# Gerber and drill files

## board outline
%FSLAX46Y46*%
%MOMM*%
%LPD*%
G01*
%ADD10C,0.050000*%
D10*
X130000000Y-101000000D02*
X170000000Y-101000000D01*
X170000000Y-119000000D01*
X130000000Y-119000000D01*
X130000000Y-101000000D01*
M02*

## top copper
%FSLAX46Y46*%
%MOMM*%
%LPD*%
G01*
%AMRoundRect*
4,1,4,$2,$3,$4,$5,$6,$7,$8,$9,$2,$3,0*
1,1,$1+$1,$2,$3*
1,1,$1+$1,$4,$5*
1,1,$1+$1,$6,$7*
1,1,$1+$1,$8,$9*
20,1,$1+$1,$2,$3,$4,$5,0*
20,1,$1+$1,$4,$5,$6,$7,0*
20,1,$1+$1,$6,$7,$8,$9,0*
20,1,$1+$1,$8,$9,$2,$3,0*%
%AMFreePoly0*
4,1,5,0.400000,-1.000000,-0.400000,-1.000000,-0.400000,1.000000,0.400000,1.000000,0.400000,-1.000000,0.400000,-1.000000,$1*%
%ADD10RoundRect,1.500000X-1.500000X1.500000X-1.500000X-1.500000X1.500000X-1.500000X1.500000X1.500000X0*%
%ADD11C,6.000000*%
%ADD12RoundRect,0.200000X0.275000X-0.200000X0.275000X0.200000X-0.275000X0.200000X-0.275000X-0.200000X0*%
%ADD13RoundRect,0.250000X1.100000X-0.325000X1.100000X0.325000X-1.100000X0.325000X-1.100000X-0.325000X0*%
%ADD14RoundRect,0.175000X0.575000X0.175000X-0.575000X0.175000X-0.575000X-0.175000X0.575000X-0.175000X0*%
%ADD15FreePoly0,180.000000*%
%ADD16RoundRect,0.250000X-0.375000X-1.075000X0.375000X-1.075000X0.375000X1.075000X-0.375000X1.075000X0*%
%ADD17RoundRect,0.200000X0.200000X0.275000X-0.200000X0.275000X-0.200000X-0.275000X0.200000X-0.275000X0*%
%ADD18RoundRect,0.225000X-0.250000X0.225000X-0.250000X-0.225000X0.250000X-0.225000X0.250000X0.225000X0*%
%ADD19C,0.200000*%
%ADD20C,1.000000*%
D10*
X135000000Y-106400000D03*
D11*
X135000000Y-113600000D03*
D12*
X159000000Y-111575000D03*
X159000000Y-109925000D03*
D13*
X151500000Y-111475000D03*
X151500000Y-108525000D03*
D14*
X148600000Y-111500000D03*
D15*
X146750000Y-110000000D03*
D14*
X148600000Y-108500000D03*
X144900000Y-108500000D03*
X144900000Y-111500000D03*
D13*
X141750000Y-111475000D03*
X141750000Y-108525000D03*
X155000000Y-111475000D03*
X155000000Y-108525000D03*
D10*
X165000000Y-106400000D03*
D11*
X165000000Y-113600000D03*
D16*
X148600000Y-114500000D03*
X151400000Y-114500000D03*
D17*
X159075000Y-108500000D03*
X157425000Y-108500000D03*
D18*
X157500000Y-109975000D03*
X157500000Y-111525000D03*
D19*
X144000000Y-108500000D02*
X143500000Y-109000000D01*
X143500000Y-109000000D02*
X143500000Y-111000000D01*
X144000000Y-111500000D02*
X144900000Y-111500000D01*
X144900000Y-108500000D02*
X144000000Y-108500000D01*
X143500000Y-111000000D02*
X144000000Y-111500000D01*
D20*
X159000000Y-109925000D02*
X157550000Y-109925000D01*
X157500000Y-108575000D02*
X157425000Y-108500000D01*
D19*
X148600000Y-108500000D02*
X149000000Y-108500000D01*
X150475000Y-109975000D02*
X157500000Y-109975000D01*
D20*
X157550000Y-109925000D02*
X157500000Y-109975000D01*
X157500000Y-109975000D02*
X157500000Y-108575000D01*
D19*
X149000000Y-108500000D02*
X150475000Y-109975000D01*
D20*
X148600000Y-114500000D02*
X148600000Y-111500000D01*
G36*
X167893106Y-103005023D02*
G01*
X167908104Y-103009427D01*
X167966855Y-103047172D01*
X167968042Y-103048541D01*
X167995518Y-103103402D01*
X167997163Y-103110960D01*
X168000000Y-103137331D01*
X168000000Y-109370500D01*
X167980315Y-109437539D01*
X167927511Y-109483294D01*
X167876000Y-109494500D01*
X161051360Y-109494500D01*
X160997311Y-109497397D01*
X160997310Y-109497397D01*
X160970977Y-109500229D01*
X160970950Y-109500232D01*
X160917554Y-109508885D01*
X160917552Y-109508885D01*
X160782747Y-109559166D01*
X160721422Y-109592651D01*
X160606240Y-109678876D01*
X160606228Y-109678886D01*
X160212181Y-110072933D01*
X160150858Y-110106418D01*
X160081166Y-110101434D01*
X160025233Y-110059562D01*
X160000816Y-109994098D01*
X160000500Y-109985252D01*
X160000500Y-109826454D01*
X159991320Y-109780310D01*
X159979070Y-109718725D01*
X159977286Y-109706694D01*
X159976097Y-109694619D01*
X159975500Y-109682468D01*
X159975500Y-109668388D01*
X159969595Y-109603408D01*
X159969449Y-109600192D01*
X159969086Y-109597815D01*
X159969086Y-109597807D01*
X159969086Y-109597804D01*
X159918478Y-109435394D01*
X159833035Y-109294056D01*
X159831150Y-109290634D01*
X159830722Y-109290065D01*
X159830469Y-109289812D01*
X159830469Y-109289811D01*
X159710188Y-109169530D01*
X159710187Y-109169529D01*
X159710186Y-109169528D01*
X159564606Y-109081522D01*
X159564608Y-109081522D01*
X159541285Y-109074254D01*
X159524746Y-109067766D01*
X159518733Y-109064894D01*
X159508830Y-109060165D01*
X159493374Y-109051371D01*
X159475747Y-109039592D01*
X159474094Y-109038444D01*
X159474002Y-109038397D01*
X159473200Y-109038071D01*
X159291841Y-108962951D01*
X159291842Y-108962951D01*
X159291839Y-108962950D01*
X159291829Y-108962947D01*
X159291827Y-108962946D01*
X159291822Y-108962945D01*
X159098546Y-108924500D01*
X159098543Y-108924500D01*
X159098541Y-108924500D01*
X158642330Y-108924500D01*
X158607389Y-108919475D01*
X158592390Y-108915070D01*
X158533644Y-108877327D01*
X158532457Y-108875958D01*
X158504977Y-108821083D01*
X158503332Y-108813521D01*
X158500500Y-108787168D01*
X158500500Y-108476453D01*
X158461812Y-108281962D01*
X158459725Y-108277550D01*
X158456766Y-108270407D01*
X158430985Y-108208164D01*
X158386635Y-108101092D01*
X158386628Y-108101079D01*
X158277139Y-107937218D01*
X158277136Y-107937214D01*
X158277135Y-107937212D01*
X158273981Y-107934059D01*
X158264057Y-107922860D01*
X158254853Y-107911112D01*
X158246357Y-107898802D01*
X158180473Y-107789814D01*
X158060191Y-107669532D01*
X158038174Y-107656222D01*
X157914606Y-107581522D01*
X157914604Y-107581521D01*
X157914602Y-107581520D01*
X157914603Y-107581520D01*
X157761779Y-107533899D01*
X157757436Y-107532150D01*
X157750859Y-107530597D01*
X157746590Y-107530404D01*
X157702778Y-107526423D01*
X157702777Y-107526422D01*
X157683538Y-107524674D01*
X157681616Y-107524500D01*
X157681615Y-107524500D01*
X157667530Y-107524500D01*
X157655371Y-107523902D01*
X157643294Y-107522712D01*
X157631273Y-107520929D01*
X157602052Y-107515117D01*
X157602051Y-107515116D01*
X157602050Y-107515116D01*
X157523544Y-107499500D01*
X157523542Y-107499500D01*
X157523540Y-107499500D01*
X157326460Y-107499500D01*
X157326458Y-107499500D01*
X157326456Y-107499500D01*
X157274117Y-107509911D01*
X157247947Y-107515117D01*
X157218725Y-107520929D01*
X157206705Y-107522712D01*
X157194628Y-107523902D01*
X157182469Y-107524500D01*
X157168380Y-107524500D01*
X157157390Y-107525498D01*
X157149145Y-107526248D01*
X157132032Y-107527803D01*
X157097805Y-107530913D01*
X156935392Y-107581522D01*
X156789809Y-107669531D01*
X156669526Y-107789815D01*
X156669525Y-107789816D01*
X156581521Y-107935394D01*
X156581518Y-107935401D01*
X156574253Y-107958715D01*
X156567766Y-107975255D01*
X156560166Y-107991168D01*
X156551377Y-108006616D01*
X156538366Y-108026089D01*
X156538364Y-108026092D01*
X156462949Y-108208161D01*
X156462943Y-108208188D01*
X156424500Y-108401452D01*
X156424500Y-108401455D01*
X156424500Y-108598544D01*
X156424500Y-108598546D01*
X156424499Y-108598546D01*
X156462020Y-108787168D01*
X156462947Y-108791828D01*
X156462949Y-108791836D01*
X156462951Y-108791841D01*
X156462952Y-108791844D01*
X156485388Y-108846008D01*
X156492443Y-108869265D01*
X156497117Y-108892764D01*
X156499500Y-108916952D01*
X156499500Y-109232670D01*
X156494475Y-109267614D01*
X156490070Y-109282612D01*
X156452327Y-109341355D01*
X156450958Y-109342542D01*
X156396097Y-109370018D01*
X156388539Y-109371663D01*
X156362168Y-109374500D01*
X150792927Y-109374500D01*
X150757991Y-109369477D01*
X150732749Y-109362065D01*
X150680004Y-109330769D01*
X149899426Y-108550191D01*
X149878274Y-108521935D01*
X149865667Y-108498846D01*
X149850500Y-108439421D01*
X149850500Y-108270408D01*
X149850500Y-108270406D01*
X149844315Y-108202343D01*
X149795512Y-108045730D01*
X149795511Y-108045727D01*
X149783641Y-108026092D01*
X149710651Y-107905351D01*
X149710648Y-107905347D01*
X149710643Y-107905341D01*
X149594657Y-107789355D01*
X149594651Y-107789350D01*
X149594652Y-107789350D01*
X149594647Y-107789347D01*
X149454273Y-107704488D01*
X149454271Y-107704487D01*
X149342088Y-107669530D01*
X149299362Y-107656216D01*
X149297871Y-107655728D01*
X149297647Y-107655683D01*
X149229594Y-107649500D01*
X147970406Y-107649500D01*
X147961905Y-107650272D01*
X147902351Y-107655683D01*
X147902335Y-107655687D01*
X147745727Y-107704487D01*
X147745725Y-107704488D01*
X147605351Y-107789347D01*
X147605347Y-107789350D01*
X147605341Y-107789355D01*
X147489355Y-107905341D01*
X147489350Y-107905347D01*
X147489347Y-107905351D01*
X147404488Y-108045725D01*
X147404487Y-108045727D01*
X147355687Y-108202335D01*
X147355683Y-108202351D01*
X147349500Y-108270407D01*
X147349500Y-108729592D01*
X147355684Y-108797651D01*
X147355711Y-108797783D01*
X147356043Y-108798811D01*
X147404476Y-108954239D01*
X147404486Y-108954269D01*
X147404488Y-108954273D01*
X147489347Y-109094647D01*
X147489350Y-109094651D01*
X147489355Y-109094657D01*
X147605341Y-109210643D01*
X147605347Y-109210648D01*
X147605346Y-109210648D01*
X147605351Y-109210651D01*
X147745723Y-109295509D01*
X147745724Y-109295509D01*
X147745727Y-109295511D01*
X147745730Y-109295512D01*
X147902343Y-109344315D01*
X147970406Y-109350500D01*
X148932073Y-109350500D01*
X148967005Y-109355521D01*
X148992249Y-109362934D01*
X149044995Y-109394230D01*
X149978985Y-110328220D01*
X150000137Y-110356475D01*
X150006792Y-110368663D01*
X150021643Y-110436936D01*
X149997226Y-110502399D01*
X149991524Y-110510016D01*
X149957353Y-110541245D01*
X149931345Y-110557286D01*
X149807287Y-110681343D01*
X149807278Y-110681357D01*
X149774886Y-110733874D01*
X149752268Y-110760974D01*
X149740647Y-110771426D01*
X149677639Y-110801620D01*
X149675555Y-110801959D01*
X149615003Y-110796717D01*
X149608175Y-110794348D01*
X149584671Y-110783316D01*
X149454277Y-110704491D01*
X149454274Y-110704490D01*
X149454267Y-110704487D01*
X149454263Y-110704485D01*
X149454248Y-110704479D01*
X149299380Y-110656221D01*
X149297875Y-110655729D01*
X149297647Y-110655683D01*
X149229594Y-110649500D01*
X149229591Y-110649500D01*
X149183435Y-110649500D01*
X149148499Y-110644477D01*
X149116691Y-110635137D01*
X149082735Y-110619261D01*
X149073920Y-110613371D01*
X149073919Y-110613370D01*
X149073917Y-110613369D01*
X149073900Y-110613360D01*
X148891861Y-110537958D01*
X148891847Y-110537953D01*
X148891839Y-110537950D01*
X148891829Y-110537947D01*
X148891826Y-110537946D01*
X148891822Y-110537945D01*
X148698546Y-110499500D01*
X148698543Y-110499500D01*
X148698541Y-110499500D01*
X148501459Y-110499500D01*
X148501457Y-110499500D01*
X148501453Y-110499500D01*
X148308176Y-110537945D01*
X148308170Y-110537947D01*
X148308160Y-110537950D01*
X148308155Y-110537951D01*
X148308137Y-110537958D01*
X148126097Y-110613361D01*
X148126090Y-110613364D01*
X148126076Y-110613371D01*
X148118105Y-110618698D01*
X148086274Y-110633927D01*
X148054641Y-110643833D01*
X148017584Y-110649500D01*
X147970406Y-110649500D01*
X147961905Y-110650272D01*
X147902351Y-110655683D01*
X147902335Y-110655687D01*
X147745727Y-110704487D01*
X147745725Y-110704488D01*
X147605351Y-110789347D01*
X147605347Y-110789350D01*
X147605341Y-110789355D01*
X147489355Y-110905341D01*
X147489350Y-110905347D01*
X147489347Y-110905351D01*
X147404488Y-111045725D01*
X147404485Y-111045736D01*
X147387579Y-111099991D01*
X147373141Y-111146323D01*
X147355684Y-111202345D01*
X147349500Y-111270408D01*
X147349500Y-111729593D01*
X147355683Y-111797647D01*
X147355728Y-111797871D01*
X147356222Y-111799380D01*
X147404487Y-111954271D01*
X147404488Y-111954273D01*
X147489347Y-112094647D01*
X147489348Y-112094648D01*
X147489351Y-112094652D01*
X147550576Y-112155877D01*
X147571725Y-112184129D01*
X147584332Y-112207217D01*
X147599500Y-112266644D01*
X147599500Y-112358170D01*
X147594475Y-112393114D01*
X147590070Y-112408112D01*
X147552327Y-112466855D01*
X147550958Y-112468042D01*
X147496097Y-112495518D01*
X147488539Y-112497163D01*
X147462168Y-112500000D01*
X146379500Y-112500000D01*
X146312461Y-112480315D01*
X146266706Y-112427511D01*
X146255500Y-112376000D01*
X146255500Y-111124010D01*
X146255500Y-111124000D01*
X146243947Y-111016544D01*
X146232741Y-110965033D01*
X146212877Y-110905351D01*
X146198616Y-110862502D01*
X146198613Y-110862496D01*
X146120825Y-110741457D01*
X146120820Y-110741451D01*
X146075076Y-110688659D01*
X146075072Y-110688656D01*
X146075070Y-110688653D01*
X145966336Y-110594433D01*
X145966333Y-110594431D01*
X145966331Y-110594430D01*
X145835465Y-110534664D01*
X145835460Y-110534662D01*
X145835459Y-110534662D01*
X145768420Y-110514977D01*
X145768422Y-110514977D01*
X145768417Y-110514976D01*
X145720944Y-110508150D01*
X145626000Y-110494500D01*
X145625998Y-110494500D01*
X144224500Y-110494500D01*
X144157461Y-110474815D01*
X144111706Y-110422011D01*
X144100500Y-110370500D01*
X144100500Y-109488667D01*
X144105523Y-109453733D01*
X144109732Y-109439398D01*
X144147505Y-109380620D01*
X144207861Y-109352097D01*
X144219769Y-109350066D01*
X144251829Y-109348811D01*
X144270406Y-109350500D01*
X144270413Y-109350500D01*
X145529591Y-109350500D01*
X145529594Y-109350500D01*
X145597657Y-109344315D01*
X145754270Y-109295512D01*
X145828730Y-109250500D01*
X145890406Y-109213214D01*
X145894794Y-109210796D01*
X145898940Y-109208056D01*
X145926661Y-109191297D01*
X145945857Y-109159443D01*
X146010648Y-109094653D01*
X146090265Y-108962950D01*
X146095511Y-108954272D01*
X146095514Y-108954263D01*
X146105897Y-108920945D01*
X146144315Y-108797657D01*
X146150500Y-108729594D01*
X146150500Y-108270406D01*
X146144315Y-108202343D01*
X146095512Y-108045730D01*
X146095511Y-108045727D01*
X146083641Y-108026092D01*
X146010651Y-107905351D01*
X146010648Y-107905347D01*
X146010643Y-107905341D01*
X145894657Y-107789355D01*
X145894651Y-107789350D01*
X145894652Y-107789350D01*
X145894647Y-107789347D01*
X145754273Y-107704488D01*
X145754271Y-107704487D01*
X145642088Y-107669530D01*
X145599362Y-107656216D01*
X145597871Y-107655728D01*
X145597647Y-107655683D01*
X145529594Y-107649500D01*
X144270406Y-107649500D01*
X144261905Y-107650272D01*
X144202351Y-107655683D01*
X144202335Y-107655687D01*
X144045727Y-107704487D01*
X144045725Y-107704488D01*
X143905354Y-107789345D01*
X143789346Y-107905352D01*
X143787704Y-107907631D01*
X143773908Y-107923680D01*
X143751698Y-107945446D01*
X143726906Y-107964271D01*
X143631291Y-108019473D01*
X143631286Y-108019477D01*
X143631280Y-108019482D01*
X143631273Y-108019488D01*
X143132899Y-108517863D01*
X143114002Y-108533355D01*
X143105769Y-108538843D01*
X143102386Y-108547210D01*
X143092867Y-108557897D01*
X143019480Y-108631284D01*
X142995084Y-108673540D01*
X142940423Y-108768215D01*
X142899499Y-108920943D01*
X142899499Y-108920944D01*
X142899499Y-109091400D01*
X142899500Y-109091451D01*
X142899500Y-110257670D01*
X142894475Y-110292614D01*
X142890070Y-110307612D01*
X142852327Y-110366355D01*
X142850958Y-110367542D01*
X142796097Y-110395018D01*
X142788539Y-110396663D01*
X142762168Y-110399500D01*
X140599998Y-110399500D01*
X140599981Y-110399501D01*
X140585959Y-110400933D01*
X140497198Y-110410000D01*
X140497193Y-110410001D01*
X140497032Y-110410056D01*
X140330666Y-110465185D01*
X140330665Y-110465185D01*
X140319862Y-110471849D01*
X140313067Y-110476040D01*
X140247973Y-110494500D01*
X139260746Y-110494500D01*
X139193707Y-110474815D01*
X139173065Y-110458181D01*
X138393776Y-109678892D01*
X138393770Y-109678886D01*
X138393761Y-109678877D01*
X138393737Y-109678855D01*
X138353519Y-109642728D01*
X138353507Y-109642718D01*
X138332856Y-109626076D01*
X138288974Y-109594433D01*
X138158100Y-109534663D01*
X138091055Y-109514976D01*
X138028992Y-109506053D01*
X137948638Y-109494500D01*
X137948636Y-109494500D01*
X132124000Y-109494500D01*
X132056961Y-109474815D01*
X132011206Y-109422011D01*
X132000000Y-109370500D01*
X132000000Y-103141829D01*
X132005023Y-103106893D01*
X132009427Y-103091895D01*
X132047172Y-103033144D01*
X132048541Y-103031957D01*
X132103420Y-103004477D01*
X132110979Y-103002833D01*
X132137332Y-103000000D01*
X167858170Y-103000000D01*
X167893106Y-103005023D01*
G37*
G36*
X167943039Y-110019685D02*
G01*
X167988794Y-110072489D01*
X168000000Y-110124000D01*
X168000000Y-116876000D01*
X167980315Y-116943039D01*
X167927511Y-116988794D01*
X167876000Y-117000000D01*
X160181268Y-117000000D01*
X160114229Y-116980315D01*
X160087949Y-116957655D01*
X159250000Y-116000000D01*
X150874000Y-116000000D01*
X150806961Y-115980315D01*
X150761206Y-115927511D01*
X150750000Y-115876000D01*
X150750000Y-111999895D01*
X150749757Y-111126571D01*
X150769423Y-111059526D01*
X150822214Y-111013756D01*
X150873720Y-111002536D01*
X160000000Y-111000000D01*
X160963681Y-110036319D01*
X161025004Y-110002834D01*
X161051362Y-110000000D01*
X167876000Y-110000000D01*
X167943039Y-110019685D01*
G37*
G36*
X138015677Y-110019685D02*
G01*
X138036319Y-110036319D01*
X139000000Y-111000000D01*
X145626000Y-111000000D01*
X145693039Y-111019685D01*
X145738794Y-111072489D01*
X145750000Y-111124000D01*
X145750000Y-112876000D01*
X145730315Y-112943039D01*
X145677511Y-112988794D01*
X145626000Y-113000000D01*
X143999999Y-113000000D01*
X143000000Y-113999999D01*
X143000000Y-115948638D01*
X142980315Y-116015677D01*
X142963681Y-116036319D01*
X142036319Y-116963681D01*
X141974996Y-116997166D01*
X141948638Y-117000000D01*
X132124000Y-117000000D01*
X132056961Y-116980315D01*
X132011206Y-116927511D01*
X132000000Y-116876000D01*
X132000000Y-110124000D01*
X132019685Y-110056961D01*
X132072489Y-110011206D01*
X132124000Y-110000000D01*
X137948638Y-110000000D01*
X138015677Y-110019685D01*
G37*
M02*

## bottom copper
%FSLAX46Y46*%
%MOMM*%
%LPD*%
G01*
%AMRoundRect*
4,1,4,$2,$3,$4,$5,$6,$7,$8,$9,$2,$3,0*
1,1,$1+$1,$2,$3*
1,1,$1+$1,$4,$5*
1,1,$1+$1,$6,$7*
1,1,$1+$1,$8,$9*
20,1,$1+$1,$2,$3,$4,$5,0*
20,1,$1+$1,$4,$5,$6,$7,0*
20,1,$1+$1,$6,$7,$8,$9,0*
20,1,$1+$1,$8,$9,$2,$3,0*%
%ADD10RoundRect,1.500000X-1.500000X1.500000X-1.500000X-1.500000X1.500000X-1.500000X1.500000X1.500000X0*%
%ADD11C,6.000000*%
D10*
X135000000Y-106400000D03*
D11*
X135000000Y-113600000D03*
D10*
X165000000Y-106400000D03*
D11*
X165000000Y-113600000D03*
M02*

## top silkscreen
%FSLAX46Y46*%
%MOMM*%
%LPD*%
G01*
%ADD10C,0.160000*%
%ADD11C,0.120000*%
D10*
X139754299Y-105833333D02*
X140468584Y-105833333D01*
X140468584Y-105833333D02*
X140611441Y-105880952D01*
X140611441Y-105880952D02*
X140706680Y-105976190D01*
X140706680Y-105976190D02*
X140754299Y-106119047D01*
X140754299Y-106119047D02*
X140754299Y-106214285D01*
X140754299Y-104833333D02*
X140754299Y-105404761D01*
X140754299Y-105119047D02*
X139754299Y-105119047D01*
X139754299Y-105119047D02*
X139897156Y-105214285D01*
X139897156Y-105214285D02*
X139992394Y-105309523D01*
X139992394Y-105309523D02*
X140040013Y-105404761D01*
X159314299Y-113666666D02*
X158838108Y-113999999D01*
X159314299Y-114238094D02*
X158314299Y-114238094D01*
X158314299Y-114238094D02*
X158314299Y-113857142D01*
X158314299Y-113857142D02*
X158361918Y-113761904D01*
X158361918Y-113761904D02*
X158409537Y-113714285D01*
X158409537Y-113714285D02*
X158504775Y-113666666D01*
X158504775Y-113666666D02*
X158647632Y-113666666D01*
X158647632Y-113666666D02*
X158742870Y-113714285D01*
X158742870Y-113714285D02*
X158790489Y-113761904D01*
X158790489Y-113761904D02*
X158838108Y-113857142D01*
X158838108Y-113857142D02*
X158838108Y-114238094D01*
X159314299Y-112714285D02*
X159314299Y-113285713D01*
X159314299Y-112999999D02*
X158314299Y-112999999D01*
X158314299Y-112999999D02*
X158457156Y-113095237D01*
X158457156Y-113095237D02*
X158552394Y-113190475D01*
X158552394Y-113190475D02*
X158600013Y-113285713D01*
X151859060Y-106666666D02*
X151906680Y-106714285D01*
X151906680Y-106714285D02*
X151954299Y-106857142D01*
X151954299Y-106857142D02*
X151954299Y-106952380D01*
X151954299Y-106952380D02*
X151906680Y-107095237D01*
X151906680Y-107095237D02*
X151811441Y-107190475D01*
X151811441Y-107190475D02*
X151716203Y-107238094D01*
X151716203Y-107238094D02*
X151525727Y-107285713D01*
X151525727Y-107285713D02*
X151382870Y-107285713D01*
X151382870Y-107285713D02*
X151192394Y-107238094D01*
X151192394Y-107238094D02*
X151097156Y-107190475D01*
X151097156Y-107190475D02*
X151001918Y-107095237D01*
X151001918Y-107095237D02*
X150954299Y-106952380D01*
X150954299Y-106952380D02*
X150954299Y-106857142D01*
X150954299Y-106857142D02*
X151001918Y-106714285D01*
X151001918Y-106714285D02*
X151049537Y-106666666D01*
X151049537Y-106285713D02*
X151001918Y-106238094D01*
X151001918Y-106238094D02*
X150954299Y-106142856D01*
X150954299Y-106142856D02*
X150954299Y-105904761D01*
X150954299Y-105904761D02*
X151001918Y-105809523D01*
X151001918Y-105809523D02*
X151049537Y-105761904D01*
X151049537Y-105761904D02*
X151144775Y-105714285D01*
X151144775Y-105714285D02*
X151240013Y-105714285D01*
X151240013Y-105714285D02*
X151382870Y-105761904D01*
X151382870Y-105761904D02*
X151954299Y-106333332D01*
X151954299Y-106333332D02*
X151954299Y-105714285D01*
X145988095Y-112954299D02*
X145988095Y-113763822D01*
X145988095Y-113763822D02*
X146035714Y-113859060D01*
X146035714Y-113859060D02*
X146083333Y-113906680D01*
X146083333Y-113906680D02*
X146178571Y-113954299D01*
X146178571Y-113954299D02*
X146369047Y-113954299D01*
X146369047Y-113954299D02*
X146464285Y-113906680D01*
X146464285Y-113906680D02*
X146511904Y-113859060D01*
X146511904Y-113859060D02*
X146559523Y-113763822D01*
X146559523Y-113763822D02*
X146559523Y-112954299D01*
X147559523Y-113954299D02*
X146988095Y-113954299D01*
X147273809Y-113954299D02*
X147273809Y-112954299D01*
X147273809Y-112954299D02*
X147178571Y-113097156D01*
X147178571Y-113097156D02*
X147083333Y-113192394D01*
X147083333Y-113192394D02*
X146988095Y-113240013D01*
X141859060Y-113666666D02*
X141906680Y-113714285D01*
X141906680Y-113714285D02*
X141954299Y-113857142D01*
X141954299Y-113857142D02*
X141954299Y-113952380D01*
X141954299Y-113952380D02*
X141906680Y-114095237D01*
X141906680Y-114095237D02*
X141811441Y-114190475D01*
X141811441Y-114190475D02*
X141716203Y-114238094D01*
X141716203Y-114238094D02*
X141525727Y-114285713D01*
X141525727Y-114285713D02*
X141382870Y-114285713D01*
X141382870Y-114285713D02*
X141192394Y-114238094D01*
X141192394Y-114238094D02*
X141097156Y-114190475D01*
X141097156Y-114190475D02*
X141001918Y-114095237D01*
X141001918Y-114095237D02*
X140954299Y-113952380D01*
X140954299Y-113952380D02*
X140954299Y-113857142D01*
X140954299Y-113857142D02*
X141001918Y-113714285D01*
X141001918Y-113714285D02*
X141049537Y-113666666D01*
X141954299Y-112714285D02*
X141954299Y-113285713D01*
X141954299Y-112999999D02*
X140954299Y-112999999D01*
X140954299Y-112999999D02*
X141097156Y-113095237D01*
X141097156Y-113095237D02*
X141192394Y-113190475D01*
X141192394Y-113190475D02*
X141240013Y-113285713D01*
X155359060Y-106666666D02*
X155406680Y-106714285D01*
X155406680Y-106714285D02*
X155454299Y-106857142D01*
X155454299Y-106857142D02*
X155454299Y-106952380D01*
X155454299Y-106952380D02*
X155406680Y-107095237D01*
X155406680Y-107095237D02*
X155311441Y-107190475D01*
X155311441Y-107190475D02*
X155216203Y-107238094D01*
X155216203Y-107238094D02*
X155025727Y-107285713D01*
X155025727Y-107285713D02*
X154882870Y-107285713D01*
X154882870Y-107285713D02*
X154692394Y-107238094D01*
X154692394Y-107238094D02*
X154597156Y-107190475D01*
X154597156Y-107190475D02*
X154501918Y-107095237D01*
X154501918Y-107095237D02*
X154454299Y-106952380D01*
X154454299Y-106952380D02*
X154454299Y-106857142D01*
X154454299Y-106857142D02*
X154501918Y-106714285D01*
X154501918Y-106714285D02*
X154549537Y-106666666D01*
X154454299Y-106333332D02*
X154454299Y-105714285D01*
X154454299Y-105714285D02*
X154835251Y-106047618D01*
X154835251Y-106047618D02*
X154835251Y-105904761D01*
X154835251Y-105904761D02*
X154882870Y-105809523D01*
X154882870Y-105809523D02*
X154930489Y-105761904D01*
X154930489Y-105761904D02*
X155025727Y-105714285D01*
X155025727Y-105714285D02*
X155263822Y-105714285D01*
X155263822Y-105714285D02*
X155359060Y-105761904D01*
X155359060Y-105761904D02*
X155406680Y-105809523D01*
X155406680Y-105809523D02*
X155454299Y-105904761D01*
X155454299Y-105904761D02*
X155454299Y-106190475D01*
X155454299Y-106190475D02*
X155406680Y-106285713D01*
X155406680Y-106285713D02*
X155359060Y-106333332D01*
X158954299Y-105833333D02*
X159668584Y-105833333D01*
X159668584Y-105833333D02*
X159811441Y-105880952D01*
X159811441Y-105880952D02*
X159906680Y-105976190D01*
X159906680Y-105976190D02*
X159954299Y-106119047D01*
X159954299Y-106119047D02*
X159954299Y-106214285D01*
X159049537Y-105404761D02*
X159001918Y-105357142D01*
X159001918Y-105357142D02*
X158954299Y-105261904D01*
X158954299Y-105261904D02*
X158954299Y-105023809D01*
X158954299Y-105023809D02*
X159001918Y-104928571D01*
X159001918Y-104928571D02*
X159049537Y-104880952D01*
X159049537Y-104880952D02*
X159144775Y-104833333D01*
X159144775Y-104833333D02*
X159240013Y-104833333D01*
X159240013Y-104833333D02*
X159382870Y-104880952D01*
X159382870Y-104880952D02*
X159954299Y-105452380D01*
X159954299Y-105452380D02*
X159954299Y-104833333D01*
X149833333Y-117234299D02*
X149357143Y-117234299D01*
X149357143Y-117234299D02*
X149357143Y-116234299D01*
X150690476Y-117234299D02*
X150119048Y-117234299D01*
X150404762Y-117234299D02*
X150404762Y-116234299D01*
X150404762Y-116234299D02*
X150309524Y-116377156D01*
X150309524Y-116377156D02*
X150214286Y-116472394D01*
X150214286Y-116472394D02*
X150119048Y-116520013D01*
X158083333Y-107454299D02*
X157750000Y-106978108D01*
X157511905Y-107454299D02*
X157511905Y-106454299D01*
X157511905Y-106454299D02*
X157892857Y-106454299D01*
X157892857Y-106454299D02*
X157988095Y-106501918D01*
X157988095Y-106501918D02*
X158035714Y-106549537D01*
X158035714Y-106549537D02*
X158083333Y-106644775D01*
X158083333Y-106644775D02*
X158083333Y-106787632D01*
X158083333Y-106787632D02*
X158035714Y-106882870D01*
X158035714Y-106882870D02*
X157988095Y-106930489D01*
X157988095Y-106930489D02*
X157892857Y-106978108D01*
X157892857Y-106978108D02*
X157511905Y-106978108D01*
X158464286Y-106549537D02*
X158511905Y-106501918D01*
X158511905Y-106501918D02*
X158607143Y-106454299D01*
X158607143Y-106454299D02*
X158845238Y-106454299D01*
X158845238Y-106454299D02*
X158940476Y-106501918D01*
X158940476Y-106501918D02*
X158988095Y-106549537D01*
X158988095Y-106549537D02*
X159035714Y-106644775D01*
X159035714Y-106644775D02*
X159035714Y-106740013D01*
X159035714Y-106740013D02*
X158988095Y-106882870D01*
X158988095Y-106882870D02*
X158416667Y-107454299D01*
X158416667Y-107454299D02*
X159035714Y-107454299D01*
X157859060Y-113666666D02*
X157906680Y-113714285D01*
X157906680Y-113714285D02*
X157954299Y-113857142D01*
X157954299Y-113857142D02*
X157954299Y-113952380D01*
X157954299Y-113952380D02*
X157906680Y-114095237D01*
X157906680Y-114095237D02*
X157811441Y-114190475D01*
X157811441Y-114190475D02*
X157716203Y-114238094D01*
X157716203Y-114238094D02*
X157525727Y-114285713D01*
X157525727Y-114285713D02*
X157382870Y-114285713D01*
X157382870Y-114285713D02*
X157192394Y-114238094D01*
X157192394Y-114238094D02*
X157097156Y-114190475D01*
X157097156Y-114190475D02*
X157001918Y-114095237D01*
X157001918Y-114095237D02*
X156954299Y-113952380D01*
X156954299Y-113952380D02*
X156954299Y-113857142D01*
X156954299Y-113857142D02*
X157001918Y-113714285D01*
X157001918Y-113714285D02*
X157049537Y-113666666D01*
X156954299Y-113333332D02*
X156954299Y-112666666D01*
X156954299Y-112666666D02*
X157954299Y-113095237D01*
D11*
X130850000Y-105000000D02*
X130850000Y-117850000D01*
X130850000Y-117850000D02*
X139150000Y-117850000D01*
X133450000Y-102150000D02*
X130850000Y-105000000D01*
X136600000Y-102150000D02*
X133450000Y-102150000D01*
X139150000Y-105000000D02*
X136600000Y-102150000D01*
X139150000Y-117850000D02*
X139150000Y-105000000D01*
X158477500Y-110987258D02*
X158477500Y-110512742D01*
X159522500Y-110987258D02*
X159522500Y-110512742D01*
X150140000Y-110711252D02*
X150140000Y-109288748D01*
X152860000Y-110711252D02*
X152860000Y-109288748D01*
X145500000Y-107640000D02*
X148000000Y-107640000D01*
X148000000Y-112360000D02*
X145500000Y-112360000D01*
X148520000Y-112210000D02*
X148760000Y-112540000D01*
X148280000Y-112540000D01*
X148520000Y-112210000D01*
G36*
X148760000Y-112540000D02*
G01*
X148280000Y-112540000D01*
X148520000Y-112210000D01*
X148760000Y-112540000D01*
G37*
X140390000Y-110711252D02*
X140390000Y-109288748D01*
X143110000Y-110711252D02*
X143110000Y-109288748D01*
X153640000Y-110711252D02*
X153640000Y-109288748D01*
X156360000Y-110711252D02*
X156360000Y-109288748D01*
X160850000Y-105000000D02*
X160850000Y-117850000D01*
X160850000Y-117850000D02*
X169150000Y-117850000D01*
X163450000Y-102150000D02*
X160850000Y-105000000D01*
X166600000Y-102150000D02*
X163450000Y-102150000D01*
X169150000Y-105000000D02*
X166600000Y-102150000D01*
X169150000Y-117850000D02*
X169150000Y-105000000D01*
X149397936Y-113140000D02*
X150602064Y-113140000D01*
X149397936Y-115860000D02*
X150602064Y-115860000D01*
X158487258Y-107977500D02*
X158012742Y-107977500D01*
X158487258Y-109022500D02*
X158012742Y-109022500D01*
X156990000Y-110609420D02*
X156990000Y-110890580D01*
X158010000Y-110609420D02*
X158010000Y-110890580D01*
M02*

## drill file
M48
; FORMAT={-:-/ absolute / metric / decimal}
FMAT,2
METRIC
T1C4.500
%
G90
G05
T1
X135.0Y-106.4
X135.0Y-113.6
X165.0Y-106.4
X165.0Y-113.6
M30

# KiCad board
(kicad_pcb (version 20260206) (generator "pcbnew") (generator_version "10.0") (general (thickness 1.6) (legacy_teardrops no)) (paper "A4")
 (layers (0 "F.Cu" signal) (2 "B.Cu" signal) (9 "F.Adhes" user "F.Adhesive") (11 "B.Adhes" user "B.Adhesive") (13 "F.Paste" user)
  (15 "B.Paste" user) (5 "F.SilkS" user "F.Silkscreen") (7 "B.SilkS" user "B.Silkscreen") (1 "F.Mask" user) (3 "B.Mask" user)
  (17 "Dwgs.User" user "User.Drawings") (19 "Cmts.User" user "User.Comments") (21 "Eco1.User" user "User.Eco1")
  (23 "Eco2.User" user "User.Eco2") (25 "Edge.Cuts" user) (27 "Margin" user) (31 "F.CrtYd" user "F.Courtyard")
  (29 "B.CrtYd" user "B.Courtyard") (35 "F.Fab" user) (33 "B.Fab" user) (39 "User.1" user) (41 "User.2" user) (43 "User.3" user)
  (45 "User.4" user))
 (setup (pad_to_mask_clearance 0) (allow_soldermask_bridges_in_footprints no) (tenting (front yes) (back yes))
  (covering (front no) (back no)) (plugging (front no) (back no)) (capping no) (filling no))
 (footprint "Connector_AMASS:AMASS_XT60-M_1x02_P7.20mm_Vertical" (layer "F.Cu") (at 135 106.4 -90)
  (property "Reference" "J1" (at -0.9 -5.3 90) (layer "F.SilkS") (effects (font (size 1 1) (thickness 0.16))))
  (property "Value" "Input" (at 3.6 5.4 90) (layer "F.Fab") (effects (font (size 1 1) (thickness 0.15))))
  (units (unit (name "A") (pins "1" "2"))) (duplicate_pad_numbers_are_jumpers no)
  (fp_line (start -1.4 4.15) (end 11.45 4.15) (stroke (width 0.12) (type solid)) (layer "F.SilkS"))
  (fp_line (start 11.45 4.15) (end 11.45 -4.15) (stroke (width 0.12) (type solid)) (layer "F.SilkS"))
  (fp_line (start -4.25 1.55) (end -1.4 4.15) (stroke (width 0.12) (type solid)) (layer "F.SilkS"))
  (fp_line (start -4.25 -1.6) (end -4.25 1.55) (stroke (width 0.12) (type solid)) (layer "F.SilkS"))
  (fp_line (start -1.4 -4.15) (end -4.25 -1.6) (stroke (width 0.12) (type solid)) (layer "F.SilkS"))
  (fp_line (start 11.45 -4.15) (end -1.4 -4.15) (stroke (width 0.12) (type solid)) (layer "F.SilkS"))
  (pad "1" thru_hole roundrect (at 0 0 270) (size 6 6) (drill 4.5) (layers "*.Cu" "*.Mask") (remove_unused_layers no)
   (roundrect_rratio 0.25) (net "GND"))
  (pad "2" thru_hole circle (at 7.2 0 270) (size 6 6) (drill 4.5) (layers "*.Cu" "*.Mask") (remove_unused_layers no) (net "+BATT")))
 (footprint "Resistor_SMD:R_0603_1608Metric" (layer "F.Cu") (at 159 110.75 90)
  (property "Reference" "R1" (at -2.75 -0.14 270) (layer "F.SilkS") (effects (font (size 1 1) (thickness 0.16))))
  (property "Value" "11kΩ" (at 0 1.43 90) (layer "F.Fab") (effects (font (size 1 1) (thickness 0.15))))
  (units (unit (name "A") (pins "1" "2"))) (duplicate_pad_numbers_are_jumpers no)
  (fp_line (start -0.237258 -0.5225) (end 0.237258 -0.5225) (stroke (width 0.12) (type solid)) (layer "F.SilkS"))
  (fp_line (start -0.237258 0.5225) (end 0.237258 0.5225) (stroke (width 0.12) (type solid)) (layer "F.SilkS"))
  (pad "1" smd roundrect (at -0.825 0 90) (size 0.8 0.95) (layers "F.Cu" "F.Mask" "F.Paste") (roundrect_rratio 0.25) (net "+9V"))
  (pad "2" smd roundrect (at 0.825 0 90) (size 0.8 0.95) (layers "F.Cu" "F.Mask" "F.Paste") (roundrect_rratio 0.25) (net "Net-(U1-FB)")))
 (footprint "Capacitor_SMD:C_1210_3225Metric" (layer "F.Cu") (at 151.5 110 90)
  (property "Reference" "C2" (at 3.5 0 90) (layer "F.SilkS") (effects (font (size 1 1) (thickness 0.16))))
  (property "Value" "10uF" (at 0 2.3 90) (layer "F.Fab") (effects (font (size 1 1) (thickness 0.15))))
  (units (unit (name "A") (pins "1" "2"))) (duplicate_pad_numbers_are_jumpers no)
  (fp_line (start -0.711252 -1.36) (end 0.711252 -1.36) (stroke (width 0.12) (type solid)) (layer "F.SilkS"))
  (fp_line (start -0.711252 1.36) (end 0.711252 1.36) (stroke (width 0.12) (type solid)) (layer "F.SilkS"))
  (pad "1" smd roundrect (at -1.475 0 90) (size 1.15 2.7) (layers "F.Cu" "F.Mask" "F.Paste") (roundrect_rratio 0.217391) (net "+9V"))
  (pad "2" smd roundrect (at 1.475 0 90) (size 1.15 2.7) (layers "F.Cu" "F.Mask" "F.Paste") (roundrect_rratio 0.217391) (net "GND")))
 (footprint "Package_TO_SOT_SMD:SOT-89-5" (layer "F.Cu") (at 146.75 110 180)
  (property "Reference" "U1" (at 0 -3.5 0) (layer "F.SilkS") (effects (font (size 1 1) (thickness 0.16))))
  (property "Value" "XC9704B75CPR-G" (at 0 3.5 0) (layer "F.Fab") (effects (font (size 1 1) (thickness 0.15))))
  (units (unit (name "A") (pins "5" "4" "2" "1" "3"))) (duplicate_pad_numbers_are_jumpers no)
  (fp_line (start 1.25 2.36) (end -1.25 2.36) (stroke (width 0.12) (type solid)) (layer "F.SilkS"))
  (fp_line (start -1.25 -2.36) (end 1.25 -2.36) (stroke (width 0.12) (type solid)) (layer "F.SilkS"))
  (fp_poly
   (pts (xy -1.77 -2.21) (xy -2.01 -2.54) (xy -1.53 -2.54) (xy -1.77 -2.21)) (stroke (width 0.12) (type solid)) (fill yes) (layer "F.SilkS"))
  (pad "1" smd roundrect (at -1.85 -1.5 180) (size 1.5 0.7) (layers "F.Cu" "F.Mask" "F.Paste") (roundrect_rratio 0.25) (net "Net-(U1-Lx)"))
  (pad "2" smd custom (at 0 0 180) (size 0.8 2) (layers "F.Cu" "F.Mask" "F.Paste") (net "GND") (zone_connect 2) (thermal_bridge_angle 45)
   (options (clearance outline) (anchor rect)) (primitives))
  (pad "3" smd roundrect (at -1.85 1.5 180) (size 1.5 0.7) (layers "F.Cu" "F.Mask" "F.Paste") (roundrect_rratio 0.25) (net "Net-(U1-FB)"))
  (pad "4" smd roundrect (at 1.85 1.5 180) (size 1.5 0.7) (layers "F.Cu" "F.Mask" "F.Paste") (roundrect_rratio 0.25) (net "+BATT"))
  (pad "5" smd roundrect (at 1.85 -1.5 180) (size 1.5 0.7) (layers "F.Cu" "F.Mask" "F.Paste") (roundrect_rratio 0.25) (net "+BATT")))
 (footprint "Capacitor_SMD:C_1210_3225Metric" (layer "F.Cu") (at 141.75 110 90)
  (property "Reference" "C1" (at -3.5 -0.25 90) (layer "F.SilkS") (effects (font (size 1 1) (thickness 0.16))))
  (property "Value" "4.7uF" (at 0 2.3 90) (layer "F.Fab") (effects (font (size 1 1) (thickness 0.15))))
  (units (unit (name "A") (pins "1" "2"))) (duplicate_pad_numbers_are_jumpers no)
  (fp_line (start -0.711252 -1.36) (end 0.711252 -1.36) (stroke (width 0.12) (type solid)) (layer "F.SilkS"))
  (fp_line (start -0.711252 1.36) (end 0.711252 1.36) (stroke (width 0.12) (type solid)) (layer "F.SilkS"))
  (pad "1" smd roundrect (at -1.475 0 90) (size 1.15 2.7) (layers "F.Cu" "F.Mask" "F.Paste") (roundrect_rratio 0.217391) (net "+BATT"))
  (pad "2" smd roundrect (at 1.475 0 90) (size 1.15 2.7) (layers "F.Cu" "F.Mask" "F.Paste") (roundrect_rratio 0.217391) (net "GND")))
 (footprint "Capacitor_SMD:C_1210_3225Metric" (layer "F.Cu") (at 155 110 90)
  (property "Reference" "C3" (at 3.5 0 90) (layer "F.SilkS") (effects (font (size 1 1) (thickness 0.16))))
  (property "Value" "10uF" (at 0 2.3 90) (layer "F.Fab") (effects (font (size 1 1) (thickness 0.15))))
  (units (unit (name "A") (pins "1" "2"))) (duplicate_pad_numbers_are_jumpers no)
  (fp_line (start -0.711252 -1.36) (end 0.711252 -1.36) (stroke (width 0.12) (type solid)) (layer "F.SilkS"))
  (fp_line (start -0.711252 1.36) (end 0.711252 1.36) (stroke (width 0.12) (type solid)) (layer "F.SilkS"))
  (pad "1" smd roundrect (at -1.475 0 90) (size 1.15 2.7) (layers "F.Cu" "F.Mask" "F.Paste") (roundrect_rratio 0.217391) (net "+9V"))
  (pad "2" smd roundrect (at 1.475 0 90) (size 1.15 2.7) (layers "F.Cu" "F.Mask" "F.Paste") (roundrect_rratio 0.217391) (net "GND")))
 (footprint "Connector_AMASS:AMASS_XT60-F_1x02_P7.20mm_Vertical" (layer "F.Cu") (at 165 106.4 -90)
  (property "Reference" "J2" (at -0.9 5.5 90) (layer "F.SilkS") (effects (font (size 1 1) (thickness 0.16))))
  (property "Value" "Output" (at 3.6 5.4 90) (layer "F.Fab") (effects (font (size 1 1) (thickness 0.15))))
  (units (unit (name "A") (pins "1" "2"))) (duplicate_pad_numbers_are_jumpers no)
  (fp_line (start -1.4 4.15) (end 11.45 4.15) (stroke (width 0.12) (type solid)) (layer "F.SilkS"))
  (fp_line (start 11.45 4.15) (end 11.45 -4.15) (stroke (width 0.12) (type solid)) (layer "F.SilkS"))
  (fp_line (start -4.25 1.55) (end -1.4 4.15) (stroke (width 0.12) (type solid)) (layer "F.SilkS"))
  (fp_line (start -4.25 -1.6) (end -4.25 1.55) (stroke (width 0.12) (type solid)) (layer "F.SilkS"))
  (fp_line (start -1.4 -4.15) (end -4.25 -1.6) (stroke (width 0.12) (type solid)) (layer "F.SilkS"))
  (fp_line (start 11.45 -4.15) (end -1.4 -4.15) (stroke (width 0.12) (type solid)) (layer "F.SilkS"))
  (pad "1" thru_hole roundrect (at 0 0 270) (size 6 6) (drill 4.5) (layers "*.Cu" "*.Mask") (remove_unused_layers no)
   (roundrect_rratio 0.25) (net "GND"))
  (pad "2" thru_hole circle (at 7.2 0 270) (size 6 6) (drill 4.5) (layers "*.Cu" "*.Mask") (remove_unused_layers no) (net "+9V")))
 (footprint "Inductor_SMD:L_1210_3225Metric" (layer "F.Cu") (at 150 114.5)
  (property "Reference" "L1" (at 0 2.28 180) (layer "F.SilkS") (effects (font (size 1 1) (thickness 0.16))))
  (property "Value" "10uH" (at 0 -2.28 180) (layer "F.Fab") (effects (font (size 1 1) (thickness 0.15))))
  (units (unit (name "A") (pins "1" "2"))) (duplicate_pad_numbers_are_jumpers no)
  (fp_line (start -0.602064 -1.36) (end 0.602064 -1.36) (stroke (width 0.12) (type solid)) (layer "F.SilkS"))
  (fp_line (start -0.602064 1.36) (end 0.602064 1.36) (stroke (width 0.12) (type solid)) (layer "F.SilkS"))
  (pad "1" smd roundrect (at -1.4 0) (size 1.25 2.65) (layers "F.Cu" "F.Mask" "F.Paste") (roundrect_rratio 0.2) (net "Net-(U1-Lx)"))
  (pad "2" smd roundrect (at 1.4 0) (size 1.25 2.65) (layers "F.Cu" "F.Mask" "F.Paste") (roundrect_rratio 0.2) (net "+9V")))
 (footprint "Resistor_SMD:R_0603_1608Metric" (layer "F.Cu") (at 158.25 108.5 180)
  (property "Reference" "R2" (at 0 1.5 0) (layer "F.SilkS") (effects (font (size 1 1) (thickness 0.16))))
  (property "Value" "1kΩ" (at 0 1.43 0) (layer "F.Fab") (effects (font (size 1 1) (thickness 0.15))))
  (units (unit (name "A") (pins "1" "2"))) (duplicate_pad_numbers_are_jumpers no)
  (fp_line (start -0.237258 0.5225) (end 0.237258 0.5225) (stroke (width 0.12) (type solid)) (layer "F.SilkS"))
  (fp_line (start -0.237258 -0.5225) (end 0.237258 -0.5225) (stroke (width 0.12) (type solid)) (layer "F.SilkS"))
  (pad "1" smd roundrect (at -0.825 0 180) (size 0.8 0.95) (layers "F.Cu" "F.Mask" "F.Paste") (roundrect_rratio 0.25) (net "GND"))
  (pad "2" smd roundrect (at 0.825 0 180) (size 0.8 0.95) (layers "F.Cu" "F.Mask" "F.Paste") (roundrect_rratio 0.25) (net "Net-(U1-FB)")))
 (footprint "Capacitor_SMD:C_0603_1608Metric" (layer "F.Cu") (at 157.5 110.75 -90)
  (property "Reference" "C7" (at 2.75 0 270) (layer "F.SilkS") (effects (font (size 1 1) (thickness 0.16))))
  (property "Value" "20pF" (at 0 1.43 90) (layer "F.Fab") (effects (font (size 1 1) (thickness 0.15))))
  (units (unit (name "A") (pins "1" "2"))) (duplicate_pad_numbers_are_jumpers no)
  (fp_line (start -0.14058 0.51) (end 0.14058 0.51) (stroke (width 0.12) (type solid)) (layer "F.SilkS"))
  (fp_line (start -0.14058 -0.51) (end 0.14058 -0.51) (stroke (width 0.12) (type solid)) (layer "F.SilkS"))
  (pad "1" smd roundrect (at -0.775 0 270) (size 0.9 0.95) (layers "F.Cu" "F.Mask" "F.Paste") (roundrect_rratio 0.25) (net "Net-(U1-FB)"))
  (pad "2" smd roundrect (at 0.775 0 270) (size 0.9 0.95) (layers "F.Cu" "F.Mask" "F.Paste") (roundrect_rratio 0.25) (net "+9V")))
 (gr_rect (start 130 101) (end 170 119) (stroke (width 0.05) (type default)) (fill no) (layer "Edge.Cuts"))
 (segment (start 144 108.5) (end 143.5 109) (width 0.2) (layer "F.Cu") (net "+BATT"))
 (segment (start 143.5 109) (end 143.5 111) (width 0.2) (layer "F.Cu") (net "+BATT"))
 (segment (start 144 111.5) (end 144.9 111.5) (width 0.2) (layer "F.Cu") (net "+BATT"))
 (segment (start 144.9 108.5) (end 144 108.5) (width 0.2) (layer "F.Cu") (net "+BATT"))
 (segment (start 143.5 111) (end 144 111.5) (width 0.2) (layer "F.Cu") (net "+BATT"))
 (segment (start 159 109.925) (end 157.55 109.925) (width 1) (layer "F.Cu") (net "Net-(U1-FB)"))
 (segment (start 157.5 108.575) (end 157.425 108.5) (width 1) (layer "F.Cu") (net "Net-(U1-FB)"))
 (segment (start 148.6 108.5) (end 149 108.5) (width 0.2) (layer "F.Cu") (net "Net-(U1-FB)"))
 (segment (start 150.475 109.975) (end 157.5 109.975) (width 0.2) (layer "F.Cu") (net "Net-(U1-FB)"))
 (segment (start 157.55 109.925) (end 157.5 109.975) (width 1) (layer "F.Cu") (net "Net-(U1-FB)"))
 (segment (start 157.5 109.975) (end 157.5 108.575) (width 1) (layer "F.Cu") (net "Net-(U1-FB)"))
 (segment (start 149 108.5) (end 150.475 109.975) (width 0.2) (layer "F.Cu") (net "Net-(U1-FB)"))
 (segment (start 148.6 114.5) (end 148.6 111.5) (width 1) (layer "F.Cu") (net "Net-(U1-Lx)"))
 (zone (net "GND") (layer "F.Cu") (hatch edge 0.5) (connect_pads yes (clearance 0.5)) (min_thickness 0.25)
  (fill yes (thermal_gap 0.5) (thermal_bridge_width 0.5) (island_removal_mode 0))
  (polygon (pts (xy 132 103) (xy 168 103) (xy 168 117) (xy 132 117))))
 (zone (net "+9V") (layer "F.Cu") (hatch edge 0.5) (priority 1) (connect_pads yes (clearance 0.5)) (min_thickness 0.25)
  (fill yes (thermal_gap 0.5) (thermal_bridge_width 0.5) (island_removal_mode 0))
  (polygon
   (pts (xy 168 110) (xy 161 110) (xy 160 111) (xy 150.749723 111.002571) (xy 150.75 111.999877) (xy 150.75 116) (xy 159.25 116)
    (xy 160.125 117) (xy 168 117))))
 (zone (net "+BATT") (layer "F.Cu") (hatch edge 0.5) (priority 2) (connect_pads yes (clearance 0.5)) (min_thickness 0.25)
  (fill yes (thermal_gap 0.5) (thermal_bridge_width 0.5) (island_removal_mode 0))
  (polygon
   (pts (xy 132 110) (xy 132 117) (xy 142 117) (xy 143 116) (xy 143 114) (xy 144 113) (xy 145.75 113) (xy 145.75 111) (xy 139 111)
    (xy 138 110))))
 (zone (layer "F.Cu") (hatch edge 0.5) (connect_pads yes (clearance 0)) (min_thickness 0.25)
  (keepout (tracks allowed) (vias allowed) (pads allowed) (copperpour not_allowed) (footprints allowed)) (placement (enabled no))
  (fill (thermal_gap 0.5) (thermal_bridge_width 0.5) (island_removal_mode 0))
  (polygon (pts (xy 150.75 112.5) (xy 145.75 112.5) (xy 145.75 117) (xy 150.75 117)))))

